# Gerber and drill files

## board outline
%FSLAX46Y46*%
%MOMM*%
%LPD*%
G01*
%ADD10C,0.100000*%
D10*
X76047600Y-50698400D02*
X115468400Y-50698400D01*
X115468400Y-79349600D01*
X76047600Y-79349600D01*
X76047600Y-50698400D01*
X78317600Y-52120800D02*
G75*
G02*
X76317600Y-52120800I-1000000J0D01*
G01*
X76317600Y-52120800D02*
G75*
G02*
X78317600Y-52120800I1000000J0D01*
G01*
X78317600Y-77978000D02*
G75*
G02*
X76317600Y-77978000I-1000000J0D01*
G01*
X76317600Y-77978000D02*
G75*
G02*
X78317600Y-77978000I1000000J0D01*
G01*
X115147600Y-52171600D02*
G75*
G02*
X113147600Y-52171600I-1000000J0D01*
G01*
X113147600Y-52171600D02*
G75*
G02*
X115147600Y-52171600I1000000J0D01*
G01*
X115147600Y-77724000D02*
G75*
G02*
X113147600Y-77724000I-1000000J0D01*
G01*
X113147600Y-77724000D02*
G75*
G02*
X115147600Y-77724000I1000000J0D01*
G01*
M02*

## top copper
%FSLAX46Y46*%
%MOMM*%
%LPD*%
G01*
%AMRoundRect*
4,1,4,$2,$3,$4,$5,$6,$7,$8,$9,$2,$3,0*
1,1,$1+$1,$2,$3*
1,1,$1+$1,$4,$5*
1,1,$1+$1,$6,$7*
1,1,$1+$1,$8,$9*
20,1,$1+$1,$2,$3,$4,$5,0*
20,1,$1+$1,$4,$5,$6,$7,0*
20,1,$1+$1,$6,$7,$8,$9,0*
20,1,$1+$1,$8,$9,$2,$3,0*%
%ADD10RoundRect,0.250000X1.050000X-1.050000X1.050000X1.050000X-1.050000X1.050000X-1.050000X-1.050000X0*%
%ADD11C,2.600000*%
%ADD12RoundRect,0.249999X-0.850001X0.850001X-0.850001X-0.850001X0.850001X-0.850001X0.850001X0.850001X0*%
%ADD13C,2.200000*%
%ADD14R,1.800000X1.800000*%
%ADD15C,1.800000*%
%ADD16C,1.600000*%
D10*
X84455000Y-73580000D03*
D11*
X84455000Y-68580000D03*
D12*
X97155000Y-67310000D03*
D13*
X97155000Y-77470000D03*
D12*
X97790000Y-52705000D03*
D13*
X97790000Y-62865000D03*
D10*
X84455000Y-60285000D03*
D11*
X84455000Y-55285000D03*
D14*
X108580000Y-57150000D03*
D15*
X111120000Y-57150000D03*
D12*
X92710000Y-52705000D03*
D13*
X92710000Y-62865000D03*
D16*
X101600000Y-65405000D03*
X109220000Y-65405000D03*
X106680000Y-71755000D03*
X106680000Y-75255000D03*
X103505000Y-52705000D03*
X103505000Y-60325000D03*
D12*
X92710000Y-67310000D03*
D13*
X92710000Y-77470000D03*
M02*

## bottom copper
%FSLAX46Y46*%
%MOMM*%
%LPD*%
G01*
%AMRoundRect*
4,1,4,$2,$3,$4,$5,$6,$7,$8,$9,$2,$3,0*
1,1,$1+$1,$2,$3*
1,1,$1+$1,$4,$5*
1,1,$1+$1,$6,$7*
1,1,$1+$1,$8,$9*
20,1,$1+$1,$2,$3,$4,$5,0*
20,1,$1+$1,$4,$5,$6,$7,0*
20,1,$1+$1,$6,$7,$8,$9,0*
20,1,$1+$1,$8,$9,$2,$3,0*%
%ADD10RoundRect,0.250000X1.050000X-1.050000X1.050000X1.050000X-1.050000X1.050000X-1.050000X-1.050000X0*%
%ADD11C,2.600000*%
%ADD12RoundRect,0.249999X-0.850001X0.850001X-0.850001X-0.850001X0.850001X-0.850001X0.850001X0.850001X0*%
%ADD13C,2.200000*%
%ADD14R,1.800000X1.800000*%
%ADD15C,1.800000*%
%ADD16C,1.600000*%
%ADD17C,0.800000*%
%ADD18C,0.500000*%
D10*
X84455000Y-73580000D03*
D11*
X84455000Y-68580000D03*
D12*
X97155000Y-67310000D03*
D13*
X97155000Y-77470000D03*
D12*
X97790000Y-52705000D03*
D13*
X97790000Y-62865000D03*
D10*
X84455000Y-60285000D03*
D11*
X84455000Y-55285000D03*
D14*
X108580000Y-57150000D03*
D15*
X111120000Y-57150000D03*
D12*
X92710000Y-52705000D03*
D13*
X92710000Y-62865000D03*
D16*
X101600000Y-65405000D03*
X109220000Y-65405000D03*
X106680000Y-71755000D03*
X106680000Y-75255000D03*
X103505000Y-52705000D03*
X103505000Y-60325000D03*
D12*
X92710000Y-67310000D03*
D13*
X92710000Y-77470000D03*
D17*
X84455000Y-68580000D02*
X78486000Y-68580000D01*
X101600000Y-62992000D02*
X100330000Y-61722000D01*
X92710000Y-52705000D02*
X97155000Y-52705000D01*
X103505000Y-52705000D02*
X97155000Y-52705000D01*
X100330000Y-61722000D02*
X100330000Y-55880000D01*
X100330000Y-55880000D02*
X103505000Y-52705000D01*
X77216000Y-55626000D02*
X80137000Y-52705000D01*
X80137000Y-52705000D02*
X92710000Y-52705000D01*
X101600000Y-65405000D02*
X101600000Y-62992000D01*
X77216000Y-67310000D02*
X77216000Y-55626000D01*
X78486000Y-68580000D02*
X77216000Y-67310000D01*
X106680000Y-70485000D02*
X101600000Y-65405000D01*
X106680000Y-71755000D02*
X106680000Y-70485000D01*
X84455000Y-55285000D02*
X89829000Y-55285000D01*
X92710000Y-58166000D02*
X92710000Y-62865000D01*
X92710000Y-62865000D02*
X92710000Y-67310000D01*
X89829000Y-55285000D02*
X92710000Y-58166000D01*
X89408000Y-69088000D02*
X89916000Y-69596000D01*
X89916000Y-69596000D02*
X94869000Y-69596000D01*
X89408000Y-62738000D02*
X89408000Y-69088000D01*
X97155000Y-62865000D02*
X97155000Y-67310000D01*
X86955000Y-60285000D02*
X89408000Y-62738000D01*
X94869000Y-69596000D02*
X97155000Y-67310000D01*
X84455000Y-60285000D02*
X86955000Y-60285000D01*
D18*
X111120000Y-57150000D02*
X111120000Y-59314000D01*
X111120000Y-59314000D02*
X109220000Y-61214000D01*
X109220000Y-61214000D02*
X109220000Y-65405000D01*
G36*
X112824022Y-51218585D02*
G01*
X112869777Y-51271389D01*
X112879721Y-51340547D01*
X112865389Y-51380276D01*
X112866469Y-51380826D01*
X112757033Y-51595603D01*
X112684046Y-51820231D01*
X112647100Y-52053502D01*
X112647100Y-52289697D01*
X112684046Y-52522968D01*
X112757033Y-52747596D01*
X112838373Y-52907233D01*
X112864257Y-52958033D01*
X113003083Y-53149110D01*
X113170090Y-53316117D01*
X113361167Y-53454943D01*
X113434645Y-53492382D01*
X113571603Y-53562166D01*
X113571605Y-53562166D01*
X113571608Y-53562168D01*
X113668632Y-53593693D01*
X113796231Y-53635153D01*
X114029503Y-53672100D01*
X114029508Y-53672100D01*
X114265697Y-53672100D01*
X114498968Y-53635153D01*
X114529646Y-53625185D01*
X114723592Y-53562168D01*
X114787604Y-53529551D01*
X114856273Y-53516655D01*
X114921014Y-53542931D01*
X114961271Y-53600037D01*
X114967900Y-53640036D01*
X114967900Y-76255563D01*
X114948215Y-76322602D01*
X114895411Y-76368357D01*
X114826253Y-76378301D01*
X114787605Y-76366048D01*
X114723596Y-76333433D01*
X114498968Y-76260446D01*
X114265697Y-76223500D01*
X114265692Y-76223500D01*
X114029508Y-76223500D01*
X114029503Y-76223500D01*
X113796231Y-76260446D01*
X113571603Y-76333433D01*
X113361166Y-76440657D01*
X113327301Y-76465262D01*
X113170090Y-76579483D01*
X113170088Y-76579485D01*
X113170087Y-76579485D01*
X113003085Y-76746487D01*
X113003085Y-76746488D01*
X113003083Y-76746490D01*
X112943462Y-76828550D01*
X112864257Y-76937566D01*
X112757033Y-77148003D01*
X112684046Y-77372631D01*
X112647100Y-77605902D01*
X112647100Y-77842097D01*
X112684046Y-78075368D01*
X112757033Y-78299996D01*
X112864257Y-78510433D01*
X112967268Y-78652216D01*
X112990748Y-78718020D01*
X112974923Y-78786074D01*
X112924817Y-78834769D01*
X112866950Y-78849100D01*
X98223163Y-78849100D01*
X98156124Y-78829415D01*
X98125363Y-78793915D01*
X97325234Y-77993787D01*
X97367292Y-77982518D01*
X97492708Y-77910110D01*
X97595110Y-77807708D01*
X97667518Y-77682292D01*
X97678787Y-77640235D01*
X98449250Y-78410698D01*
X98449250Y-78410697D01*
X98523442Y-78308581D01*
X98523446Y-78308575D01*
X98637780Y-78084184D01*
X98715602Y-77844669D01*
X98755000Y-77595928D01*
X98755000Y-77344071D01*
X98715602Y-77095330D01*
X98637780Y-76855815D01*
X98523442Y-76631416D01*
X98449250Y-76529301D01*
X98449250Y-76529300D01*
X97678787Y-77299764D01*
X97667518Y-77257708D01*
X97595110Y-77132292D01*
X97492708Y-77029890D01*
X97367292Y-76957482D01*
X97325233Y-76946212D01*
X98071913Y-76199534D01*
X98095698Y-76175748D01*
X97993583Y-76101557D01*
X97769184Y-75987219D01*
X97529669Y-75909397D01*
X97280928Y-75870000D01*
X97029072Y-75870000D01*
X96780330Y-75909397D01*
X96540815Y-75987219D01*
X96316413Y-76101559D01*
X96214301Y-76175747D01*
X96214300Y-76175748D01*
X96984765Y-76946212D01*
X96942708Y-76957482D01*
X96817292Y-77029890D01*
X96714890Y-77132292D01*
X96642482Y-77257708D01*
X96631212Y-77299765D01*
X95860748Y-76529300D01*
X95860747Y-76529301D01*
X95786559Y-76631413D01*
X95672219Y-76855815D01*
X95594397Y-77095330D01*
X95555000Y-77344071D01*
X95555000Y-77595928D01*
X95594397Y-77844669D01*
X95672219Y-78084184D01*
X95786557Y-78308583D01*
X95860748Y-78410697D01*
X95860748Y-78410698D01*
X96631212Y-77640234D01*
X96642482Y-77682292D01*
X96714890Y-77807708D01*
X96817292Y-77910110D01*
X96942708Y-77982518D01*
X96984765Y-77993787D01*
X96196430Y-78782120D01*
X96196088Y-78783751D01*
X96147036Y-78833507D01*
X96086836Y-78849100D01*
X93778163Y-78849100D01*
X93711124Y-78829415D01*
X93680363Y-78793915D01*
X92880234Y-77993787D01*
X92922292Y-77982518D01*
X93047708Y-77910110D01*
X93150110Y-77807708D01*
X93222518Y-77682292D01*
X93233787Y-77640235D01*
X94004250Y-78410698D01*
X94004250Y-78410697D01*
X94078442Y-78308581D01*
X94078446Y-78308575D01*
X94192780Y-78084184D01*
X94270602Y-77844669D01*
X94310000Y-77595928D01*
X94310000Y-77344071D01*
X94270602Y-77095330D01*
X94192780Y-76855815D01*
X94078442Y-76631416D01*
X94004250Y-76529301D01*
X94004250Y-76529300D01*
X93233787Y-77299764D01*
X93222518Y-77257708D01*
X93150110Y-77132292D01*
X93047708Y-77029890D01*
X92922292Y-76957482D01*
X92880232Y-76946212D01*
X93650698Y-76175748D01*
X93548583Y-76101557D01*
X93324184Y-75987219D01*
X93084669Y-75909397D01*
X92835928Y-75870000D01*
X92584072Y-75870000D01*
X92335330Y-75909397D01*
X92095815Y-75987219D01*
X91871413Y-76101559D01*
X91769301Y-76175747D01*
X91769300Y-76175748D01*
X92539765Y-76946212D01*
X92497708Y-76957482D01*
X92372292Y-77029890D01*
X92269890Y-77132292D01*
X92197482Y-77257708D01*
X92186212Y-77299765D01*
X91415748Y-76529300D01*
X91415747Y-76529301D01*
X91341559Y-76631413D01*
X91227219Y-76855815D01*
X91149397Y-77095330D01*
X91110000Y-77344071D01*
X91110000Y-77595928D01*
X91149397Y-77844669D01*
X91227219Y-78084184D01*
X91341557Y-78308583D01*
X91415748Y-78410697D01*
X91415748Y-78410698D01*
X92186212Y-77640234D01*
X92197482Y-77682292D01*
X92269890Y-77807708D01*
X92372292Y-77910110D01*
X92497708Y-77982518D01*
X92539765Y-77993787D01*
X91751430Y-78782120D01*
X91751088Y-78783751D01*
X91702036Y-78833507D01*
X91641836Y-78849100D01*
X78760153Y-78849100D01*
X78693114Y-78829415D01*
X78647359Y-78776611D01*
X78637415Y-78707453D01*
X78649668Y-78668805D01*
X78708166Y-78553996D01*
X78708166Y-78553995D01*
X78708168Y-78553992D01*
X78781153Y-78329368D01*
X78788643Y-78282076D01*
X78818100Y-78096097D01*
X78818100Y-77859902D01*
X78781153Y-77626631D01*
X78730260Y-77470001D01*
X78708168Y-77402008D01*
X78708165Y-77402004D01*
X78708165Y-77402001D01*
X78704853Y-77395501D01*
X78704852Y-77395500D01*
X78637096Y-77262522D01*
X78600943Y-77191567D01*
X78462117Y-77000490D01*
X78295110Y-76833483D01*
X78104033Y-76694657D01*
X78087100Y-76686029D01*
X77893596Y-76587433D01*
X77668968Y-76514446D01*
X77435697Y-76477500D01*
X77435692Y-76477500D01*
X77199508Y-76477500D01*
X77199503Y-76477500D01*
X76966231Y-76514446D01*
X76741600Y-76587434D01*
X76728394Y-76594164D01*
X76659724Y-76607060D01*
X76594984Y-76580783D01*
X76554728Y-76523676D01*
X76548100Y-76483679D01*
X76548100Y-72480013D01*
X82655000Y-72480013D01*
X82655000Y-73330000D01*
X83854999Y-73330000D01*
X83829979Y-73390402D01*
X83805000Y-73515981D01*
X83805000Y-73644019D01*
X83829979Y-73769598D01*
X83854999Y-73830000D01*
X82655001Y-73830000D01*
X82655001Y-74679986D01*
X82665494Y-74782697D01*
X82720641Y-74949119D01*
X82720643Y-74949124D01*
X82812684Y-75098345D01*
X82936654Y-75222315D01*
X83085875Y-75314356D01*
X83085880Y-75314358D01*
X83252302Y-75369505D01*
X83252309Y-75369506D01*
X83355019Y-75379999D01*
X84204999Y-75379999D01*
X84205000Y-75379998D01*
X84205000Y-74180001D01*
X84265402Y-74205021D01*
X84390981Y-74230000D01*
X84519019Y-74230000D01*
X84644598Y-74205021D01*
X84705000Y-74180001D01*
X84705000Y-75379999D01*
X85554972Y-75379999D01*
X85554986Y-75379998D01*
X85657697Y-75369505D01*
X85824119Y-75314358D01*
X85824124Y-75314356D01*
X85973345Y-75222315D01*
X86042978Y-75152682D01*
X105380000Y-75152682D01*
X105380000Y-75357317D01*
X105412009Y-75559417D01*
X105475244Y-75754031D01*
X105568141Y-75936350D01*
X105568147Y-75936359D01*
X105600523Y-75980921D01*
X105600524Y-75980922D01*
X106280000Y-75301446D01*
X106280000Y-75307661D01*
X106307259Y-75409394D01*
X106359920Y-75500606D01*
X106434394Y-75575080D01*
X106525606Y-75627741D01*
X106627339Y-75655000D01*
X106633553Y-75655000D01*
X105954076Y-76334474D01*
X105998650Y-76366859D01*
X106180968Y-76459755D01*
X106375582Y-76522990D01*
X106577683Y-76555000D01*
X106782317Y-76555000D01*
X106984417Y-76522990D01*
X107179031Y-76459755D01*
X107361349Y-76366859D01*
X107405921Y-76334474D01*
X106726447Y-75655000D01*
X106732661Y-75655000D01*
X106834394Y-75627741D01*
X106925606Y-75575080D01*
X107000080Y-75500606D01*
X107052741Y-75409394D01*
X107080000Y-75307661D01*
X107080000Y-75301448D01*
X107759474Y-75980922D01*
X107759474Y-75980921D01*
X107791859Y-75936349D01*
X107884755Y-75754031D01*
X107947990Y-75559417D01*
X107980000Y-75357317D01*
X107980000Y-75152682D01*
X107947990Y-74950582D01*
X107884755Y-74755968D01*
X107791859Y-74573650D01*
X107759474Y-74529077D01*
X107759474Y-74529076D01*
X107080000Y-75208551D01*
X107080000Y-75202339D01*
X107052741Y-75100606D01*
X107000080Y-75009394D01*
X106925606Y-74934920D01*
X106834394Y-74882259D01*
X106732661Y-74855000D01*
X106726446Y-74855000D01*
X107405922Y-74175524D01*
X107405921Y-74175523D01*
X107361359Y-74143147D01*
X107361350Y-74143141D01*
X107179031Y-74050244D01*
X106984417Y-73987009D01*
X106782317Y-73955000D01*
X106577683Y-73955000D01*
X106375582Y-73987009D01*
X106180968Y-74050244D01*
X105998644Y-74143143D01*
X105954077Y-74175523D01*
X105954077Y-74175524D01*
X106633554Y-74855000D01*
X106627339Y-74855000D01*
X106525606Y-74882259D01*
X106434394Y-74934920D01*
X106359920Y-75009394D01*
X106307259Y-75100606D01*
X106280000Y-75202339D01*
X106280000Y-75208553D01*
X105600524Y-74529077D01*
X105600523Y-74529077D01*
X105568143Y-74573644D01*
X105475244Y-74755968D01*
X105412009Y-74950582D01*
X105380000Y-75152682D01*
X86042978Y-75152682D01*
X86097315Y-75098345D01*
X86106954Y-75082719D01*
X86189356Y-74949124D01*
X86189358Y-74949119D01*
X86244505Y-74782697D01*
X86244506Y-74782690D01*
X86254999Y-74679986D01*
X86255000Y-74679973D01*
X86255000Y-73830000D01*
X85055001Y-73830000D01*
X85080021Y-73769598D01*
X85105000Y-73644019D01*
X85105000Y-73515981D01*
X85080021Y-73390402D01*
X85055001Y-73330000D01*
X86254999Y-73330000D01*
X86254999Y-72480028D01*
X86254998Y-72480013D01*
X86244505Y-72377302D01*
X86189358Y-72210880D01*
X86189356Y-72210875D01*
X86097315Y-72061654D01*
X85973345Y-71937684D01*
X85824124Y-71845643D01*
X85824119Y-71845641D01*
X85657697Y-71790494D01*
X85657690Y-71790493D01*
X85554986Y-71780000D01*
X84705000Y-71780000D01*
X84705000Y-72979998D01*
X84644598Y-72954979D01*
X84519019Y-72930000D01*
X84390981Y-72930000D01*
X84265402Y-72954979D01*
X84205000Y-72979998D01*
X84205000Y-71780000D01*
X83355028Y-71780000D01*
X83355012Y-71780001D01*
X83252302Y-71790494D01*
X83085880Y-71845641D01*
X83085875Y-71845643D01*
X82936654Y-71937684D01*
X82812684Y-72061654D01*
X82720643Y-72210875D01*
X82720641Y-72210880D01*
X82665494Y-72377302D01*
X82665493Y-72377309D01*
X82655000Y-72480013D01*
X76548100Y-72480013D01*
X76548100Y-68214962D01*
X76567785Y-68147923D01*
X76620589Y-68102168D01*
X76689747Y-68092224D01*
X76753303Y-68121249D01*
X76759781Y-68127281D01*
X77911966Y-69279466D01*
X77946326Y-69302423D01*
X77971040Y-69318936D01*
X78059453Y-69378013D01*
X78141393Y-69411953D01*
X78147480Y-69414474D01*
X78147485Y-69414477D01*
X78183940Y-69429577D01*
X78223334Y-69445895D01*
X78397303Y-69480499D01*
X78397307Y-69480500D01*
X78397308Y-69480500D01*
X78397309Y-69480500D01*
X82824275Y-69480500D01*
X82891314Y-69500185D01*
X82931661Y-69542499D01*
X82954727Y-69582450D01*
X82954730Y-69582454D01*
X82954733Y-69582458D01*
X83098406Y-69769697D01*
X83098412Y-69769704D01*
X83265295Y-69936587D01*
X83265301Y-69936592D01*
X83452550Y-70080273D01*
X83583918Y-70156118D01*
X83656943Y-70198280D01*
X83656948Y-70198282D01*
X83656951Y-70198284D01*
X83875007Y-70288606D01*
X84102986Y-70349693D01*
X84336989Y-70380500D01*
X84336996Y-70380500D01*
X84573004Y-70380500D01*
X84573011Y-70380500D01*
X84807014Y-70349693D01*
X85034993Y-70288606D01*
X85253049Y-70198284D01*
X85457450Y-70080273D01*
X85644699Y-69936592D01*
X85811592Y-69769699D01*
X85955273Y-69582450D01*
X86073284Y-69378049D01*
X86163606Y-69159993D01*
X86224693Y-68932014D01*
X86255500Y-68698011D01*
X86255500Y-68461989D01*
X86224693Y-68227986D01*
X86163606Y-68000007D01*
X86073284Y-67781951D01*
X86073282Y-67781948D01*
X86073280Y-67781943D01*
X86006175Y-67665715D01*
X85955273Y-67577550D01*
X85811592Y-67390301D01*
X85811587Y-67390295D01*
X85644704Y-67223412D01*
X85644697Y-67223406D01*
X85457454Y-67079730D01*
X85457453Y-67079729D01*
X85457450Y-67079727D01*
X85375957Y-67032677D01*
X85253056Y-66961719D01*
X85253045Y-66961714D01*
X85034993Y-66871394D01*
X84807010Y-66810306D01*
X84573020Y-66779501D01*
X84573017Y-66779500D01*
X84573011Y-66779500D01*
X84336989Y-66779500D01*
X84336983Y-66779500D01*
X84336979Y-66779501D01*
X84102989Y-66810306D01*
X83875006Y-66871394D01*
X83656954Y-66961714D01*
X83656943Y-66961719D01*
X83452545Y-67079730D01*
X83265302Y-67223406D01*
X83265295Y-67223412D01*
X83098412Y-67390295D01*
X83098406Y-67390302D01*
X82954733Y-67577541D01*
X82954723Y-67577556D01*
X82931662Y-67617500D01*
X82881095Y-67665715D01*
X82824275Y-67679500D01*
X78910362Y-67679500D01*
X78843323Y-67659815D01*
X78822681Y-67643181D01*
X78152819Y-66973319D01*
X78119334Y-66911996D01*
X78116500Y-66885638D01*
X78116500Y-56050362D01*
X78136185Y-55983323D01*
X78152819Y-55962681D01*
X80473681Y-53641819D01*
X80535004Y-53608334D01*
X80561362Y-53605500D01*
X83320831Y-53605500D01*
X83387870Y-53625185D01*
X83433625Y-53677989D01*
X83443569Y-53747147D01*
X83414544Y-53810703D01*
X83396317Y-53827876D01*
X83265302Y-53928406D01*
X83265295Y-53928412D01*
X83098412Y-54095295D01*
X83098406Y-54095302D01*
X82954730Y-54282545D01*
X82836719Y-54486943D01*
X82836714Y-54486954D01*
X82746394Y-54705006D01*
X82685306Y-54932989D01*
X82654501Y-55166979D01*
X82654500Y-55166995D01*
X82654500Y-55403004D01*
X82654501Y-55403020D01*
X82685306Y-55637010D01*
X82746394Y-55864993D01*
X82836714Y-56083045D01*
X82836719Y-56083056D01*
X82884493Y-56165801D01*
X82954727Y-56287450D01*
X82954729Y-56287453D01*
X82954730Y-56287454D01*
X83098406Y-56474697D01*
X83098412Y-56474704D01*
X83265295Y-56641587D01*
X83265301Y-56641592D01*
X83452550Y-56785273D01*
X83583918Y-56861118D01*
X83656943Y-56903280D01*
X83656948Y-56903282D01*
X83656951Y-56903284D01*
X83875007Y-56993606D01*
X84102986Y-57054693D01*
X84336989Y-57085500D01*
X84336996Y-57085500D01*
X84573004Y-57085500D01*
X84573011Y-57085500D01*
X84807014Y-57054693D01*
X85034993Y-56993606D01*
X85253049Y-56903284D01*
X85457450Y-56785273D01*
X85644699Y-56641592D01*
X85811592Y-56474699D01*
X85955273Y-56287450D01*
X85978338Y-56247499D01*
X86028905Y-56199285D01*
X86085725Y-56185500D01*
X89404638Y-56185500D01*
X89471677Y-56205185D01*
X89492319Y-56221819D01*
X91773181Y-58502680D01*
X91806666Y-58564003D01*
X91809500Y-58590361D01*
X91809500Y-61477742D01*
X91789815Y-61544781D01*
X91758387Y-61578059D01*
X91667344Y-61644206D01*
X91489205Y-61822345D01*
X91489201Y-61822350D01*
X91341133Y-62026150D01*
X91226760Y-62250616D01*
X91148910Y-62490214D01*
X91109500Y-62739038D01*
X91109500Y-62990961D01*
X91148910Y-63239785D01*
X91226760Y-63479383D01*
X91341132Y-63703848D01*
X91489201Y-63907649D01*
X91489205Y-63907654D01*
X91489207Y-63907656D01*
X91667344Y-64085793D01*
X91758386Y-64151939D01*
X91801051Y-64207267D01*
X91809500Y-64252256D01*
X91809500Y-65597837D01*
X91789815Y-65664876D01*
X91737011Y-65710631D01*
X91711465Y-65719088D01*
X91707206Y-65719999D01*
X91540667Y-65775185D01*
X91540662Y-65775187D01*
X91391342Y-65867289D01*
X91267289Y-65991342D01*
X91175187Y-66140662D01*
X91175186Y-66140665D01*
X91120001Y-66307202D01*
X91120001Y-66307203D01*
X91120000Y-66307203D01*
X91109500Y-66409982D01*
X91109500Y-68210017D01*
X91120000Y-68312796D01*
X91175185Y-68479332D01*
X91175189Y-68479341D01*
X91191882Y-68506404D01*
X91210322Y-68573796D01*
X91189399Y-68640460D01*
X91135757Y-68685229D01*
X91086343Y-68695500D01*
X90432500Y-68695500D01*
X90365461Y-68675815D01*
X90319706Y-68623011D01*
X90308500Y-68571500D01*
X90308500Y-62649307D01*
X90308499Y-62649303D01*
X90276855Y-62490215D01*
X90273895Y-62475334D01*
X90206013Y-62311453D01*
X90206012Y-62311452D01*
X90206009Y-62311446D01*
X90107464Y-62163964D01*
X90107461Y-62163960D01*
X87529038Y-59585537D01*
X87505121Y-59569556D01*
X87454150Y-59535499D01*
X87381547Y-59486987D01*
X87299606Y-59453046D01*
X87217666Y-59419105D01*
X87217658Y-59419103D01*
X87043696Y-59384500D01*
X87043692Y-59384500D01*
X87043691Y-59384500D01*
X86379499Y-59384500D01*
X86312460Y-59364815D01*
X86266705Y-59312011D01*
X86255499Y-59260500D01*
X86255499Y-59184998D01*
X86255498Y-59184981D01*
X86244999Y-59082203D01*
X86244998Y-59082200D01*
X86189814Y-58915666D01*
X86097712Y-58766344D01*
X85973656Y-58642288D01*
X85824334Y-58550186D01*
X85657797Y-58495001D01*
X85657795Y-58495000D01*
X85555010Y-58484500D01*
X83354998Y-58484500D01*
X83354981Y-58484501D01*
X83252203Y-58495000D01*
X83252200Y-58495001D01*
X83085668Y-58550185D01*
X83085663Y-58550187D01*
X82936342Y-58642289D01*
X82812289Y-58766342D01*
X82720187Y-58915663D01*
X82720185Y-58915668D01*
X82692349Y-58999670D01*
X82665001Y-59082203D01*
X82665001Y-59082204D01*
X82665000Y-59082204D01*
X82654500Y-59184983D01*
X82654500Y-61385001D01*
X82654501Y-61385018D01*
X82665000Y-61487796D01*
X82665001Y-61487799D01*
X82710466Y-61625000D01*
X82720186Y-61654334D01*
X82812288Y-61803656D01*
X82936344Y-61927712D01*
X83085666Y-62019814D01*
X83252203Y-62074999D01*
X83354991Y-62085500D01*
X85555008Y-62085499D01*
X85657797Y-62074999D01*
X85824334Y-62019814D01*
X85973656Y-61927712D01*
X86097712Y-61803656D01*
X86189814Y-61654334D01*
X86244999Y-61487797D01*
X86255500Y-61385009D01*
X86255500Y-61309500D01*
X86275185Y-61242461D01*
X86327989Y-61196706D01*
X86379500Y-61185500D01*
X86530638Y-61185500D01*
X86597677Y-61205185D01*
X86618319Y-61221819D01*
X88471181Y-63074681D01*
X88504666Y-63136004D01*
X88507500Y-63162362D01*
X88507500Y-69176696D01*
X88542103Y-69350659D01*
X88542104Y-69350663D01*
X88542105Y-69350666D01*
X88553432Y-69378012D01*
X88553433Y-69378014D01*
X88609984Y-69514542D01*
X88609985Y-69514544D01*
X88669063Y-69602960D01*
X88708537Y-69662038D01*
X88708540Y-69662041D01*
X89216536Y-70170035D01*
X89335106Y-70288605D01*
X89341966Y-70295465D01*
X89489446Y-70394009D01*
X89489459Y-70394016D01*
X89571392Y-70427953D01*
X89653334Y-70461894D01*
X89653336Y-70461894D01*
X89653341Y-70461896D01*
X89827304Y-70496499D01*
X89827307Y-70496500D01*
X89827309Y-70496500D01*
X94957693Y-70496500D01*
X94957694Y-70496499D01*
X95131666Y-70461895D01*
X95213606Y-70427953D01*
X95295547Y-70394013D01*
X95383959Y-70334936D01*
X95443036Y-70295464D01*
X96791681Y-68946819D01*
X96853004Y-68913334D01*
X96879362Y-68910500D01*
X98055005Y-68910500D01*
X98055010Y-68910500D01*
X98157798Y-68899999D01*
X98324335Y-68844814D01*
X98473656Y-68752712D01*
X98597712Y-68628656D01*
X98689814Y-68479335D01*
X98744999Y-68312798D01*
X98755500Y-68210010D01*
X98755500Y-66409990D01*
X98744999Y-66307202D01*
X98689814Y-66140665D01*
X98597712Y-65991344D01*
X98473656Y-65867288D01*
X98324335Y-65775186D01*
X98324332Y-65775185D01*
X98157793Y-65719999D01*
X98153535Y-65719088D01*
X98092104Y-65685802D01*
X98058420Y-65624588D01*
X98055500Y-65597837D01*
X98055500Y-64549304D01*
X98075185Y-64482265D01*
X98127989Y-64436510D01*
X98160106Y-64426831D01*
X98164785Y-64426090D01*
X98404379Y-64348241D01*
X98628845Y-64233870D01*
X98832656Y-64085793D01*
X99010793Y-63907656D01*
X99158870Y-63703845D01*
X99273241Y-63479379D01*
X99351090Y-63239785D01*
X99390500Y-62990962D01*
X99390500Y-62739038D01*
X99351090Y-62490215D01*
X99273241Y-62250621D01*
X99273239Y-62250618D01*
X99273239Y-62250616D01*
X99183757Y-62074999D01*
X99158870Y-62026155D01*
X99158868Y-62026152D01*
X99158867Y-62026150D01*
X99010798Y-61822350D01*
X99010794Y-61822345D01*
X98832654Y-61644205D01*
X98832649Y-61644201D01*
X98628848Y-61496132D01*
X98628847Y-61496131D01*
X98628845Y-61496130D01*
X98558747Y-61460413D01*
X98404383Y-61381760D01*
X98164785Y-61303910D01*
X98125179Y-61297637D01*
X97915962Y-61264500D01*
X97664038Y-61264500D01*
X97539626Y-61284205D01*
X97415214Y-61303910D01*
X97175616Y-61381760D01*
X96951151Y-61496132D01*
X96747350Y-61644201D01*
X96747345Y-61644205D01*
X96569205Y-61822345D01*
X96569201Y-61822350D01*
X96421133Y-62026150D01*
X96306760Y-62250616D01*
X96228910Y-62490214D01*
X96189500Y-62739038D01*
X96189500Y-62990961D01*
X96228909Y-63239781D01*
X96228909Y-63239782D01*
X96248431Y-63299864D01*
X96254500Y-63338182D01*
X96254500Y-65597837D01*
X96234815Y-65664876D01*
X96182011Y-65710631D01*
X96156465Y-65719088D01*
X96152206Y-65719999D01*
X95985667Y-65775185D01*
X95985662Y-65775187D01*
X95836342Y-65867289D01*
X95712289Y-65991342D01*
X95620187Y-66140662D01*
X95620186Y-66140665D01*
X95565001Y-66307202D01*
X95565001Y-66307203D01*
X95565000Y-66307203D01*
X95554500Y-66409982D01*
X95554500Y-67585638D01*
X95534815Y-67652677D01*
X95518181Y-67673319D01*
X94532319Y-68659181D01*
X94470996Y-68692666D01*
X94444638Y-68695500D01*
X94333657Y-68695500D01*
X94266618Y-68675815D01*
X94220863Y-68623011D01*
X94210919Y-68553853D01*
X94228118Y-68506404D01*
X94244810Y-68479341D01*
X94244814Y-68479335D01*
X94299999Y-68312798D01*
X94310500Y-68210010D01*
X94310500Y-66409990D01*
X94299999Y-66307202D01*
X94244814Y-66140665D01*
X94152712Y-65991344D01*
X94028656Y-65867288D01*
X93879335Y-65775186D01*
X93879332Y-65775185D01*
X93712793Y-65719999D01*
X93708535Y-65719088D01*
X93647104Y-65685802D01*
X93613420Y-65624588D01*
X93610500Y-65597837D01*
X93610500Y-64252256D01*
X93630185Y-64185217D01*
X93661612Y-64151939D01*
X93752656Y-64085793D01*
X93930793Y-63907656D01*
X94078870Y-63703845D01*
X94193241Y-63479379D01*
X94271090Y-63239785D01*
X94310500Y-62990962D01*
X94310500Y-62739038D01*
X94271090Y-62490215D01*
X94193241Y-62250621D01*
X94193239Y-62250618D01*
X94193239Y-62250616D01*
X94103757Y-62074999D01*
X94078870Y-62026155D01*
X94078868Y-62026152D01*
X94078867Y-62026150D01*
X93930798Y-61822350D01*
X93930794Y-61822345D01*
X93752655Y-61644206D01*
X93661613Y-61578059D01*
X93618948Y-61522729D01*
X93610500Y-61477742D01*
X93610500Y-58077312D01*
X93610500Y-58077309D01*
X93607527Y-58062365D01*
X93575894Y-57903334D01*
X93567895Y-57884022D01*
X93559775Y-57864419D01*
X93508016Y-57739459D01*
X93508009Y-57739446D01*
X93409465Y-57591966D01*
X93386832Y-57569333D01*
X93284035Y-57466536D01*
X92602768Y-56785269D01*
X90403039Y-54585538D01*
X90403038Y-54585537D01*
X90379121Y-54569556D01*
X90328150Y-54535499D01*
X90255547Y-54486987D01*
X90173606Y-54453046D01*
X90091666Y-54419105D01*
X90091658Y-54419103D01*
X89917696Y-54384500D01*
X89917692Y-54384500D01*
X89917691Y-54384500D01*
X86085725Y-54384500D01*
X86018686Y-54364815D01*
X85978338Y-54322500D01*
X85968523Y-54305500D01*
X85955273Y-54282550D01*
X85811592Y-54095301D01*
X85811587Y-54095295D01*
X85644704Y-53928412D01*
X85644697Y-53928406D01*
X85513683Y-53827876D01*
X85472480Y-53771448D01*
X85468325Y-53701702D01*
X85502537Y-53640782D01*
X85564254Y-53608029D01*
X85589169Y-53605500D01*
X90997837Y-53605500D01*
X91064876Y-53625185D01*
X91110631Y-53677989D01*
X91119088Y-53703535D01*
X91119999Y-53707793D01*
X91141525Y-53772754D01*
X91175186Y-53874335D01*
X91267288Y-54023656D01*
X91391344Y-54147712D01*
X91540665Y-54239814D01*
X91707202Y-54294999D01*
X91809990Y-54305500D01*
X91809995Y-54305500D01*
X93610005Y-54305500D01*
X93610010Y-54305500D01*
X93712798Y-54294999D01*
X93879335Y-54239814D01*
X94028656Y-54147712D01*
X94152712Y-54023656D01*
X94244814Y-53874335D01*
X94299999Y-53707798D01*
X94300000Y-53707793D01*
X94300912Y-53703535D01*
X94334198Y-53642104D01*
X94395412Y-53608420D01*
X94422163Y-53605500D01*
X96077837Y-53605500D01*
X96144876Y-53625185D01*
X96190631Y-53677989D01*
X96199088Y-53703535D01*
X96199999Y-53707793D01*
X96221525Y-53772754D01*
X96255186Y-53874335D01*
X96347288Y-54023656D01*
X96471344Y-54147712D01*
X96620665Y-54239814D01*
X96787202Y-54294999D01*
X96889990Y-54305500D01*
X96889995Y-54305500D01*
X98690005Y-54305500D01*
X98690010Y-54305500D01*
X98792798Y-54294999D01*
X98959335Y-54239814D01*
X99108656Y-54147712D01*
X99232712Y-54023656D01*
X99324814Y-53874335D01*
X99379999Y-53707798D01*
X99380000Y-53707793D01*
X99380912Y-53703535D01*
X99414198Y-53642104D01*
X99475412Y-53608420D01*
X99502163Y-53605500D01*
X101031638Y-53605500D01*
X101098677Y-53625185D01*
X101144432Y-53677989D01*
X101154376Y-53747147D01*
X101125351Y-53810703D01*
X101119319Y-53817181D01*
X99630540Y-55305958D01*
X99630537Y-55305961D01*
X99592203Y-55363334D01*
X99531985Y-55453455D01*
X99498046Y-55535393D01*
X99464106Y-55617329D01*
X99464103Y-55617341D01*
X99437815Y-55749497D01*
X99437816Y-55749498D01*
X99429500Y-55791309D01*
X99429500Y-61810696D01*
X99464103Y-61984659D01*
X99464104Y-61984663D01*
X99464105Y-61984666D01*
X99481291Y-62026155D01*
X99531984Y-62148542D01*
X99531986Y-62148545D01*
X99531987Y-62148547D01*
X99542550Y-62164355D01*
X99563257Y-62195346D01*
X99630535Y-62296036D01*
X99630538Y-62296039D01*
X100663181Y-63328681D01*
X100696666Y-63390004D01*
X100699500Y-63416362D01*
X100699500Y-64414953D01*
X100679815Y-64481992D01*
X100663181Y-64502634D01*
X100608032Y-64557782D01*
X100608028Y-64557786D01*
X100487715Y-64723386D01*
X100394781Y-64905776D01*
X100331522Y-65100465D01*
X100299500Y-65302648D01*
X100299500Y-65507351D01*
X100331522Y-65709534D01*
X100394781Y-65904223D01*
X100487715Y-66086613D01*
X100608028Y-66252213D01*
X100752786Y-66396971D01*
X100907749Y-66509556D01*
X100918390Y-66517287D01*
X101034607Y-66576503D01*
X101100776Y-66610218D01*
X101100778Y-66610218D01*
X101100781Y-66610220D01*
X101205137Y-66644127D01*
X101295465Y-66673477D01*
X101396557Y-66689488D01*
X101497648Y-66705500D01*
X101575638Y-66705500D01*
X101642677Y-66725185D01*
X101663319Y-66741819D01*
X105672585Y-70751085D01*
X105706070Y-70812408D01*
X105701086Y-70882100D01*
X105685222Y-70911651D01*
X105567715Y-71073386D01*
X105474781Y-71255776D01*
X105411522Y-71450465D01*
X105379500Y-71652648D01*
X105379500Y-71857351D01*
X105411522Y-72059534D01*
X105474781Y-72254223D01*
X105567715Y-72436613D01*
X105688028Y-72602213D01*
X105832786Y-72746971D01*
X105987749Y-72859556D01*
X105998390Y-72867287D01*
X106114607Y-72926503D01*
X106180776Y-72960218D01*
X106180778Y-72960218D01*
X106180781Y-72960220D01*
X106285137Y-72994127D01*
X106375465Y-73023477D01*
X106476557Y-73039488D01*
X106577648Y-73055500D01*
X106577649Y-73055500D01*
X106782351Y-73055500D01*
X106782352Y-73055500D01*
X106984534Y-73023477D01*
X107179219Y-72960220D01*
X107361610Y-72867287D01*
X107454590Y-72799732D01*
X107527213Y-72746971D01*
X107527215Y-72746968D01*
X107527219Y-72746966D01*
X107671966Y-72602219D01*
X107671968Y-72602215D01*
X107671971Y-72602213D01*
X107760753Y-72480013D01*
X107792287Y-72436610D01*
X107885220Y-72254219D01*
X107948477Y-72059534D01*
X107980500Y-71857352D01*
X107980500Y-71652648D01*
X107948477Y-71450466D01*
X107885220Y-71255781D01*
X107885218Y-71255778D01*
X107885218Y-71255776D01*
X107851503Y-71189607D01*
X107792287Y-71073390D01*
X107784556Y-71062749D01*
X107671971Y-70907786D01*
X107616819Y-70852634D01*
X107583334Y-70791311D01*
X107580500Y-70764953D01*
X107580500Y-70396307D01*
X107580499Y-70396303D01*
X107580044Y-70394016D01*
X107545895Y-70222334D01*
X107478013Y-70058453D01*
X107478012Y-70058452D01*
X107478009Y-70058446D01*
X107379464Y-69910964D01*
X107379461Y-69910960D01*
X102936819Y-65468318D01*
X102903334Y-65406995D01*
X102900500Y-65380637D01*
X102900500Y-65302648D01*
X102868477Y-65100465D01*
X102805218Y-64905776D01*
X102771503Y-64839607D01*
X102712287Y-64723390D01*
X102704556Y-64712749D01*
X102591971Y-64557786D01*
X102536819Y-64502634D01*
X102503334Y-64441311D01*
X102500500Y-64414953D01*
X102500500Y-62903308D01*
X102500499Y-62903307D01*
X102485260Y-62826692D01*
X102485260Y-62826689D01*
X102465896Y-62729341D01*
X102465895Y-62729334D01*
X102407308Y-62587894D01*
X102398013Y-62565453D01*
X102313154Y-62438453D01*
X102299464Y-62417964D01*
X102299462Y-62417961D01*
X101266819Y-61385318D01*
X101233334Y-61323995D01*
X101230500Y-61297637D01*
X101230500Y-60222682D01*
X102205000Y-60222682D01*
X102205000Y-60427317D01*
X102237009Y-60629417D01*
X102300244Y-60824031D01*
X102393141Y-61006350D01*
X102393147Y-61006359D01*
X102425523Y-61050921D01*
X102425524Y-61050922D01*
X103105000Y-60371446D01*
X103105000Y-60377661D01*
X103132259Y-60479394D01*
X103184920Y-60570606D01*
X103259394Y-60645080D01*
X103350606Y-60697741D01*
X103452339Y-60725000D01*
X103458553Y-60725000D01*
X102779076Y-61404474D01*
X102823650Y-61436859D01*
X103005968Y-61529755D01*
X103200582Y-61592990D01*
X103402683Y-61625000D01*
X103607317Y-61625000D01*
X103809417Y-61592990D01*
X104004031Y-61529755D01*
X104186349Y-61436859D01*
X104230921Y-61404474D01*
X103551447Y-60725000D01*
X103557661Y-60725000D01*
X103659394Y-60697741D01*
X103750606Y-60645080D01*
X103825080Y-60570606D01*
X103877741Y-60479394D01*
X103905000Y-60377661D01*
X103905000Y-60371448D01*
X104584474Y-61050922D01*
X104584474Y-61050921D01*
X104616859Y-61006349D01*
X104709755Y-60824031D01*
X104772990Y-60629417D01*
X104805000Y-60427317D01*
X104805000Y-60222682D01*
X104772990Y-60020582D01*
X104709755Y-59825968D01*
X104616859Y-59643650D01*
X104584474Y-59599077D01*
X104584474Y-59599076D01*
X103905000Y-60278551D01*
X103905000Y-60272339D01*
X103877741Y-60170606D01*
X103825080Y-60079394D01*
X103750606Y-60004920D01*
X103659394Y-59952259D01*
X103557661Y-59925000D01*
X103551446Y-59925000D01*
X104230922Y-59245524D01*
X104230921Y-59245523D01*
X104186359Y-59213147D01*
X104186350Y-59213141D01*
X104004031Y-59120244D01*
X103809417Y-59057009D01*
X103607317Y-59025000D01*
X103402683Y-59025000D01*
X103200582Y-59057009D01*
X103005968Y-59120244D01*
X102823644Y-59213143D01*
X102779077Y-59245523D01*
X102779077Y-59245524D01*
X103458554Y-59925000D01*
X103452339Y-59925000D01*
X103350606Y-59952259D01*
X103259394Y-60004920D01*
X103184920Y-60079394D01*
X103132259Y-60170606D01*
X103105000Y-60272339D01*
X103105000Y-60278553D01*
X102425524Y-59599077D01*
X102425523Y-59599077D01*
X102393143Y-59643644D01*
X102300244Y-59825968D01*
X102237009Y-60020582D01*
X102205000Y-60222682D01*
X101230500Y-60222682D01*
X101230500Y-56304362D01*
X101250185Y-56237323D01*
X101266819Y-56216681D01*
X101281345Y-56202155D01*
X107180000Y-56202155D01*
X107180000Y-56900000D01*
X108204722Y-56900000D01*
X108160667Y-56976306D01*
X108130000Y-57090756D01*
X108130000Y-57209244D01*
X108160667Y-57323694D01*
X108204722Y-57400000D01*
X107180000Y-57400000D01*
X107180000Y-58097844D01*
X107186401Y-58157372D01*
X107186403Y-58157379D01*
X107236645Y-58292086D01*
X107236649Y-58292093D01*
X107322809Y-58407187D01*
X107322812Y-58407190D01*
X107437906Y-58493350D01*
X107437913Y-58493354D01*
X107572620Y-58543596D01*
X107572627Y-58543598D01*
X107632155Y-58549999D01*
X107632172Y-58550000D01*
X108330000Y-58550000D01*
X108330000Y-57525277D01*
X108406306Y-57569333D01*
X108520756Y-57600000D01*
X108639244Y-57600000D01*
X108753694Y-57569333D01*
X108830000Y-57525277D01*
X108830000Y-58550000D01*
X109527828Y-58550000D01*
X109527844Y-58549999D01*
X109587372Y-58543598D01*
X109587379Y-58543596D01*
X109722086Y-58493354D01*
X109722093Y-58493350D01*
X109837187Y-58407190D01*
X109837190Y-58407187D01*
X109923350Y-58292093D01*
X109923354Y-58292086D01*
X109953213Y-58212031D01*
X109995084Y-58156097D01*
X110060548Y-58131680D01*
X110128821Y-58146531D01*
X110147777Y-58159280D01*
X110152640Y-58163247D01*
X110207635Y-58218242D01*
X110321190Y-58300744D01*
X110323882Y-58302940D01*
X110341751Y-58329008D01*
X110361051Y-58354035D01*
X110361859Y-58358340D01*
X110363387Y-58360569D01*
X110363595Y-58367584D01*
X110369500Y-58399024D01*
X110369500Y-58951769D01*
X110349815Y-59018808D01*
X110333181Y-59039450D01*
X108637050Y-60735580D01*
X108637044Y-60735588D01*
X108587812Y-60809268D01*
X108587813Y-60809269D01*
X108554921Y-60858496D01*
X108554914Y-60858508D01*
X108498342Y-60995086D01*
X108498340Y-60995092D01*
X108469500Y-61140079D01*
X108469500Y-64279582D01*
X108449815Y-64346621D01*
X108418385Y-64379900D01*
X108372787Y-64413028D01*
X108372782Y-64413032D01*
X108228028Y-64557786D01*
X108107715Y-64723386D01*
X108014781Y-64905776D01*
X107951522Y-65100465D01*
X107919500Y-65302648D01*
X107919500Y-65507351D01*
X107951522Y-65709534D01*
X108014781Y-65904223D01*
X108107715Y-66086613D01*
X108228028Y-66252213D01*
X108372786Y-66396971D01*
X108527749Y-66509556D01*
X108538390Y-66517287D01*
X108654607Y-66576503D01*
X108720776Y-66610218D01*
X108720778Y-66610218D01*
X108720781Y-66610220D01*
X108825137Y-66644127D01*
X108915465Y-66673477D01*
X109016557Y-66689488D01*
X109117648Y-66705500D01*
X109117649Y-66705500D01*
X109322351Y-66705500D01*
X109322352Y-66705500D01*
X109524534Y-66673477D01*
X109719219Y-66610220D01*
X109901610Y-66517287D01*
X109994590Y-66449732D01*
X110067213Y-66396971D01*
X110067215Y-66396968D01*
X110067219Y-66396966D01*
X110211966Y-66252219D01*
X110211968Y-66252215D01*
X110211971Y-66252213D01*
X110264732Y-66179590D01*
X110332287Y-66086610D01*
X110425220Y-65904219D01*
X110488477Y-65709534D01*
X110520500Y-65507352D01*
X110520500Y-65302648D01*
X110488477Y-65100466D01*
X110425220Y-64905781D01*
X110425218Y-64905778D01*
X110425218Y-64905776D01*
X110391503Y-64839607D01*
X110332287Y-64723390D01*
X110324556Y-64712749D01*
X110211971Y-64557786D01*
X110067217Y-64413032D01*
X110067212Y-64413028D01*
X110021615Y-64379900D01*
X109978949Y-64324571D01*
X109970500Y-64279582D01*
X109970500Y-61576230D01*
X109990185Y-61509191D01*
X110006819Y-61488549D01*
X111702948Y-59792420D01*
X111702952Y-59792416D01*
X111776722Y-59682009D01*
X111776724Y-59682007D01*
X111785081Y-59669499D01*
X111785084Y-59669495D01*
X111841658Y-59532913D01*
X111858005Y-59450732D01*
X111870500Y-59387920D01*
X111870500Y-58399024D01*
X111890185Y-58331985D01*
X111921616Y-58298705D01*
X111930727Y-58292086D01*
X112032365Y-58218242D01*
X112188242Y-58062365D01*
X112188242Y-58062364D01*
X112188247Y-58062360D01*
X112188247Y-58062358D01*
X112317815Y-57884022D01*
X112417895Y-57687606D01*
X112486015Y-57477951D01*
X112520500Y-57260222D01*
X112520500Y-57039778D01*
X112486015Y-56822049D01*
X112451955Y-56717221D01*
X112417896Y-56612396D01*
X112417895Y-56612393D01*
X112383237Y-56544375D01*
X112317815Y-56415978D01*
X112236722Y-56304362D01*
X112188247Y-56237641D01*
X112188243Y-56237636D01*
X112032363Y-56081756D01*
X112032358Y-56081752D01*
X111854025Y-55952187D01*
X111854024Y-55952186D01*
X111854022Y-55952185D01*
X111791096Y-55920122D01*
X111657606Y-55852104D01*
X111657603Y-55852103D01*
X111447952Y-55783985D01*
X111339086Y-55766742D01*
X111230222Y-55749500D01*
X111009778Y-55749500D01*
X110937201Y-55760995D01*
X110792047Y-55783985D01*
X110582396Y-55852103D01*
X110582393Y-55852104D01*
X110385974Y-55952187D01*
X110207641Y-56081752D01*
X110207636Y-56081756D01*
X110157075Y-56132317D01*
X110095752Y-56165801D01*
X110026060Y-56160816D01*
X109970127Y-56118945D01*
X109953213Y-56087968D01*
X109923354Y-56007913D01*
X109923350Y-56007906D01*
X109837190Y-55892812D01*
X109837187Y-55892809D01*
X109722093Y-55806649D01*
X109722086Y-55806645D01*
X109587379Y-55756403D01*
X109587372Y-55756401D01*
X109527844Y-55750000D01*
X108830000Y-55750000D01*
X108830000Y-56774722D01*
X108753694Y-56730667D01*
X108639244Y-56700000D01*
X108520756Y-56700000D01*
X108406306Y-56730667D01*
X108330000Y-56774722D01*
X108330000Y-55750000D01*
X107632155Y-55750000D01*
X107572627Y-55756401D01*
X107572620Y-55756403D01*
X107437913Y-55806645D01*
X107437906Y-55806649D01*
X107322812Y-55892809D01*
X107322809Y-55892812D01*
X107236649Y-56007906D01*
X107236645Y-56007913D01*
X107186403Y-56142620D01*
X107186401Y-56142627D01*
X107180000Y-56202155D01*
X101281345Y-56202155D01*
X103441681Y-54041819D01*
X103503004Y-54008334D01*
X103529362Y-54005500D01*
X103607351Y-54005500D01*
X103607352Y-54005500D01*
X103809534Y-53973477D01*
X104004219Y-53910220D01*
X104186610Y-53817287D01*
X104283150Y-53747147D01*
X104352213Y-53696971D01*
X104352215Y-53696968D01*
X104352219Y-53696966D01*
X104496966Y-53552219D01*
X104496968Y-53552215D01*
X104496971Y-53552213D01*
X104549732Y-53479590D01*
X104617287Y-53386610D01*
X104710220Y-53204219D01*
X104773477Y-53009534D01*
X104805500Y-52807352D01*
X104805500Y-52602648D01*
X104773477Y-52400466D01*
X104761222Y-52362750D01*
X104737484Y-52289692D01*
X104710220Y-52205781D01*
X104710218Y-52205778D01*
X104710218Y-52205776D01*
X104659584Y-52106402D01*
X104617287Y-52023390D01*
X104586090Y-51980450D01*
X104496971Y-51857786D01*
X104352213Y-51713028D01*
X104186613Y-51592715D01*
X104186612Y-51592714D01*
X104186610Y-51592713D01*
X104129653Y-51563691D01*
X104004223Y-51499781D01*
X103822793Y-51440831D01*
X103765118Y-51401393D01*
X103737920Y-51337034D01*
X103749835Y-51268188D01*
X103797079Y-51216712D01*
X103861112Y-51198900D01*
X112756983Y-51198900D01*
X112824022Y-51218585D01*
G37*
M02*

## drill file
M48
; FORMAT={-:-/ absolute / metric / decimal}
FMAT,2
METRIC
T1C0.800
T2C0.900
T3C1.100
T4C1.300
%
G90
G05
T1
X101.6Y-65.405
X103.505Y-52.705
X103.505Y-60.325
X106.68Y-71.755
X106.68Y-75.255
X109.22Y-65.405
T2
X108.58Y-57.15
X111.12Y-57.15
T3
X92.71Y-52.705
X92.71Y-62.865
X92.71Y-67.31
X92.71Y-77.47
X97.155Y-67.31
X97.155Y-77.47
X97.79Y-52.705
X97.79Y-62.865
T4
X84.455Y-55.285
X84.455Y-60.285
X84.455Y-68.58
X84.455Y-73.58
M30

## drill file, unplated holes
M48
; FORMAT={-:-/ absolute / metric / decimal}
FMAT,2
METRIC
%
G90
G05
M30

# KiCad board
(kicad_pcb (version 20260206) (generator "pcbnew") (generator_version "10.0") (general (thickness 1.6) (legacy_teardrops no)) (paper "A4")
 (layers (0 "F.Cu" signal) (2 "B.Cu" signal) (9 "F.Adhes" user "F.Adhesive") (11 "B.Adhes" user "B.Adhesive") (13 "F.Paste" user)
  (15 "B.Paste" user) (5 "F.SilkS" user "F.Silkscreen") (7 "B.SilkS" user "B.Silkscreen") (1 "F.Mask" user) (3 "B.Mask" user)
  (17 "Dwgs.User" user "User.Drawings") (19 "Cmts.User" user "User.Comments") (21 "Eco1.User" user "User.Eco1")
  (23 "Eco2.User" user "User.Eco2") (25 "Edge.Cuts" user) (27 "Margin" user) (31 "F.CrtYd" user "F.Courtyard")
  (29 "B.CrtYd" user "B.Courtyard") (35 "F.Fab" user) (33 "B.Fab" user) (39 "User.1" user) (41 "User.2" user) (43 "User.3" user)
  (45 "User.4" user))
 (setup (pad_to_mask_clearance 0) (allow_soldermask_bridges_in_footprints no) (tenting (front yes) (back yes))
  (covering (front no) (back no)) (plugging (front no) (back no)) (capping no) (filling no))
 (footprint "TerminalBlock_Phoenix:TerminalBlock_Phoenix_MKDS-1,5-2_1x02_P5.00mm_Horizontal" (layer "F.Cu") (at 84.455 73.58 90)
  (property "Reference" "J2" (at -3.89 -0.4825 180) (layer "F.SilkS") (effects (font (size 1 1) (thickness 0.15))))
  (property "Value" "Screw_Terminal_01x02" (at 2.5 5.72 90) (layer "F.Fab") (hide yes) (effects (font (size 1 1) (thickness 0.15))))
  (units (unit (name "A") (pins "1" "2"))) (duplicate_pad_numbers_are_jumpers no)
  (pad "1" thru_hole roundrect (at 0 0 90) (size 2.6 2.6) (drill 1.3) (layers "*.Cu" "*.Mask") (remove_unused_layers no)
   (roundrect_rratio 0.096154) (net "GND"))
  (pad "2" thru_hole circle (at 5 0 90) (size 2.6 2.6) (drill 1.3) (layers "*.Cu" "*.Mask") (remove_unused_layers no) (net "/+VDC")))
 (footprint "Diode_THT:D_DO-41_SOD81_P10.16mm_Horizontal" (layer "F.Cu") (at 97.155 67.31 -90)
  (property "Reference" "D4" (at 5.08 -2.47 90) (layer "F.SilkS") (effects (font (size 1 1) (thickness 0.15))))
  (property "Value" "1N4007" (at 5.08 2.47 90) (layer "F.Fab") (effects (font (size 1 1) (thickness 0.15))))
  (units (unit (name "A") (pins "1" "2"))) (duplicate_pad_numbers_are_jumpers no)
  (pad "1" thru_hole roundrect (at 0 0 270) (size 2.2 2.2) (drill 1.1) (layers "*.Cu" "*.Mask") (remove_unused_layers no)
   (roundrect_rratio 0.113636) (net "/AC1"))
  (pad "2" thru_hole circle (at 10.16 0 270) (size 2.2 2.2) (drill 1.1) (layers "*.Cu" "*.Mask") (remove_unused_layers no) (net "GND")))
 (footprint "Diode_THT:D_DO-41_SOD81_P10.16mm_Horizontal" (layer "F.Cu") (at 97.79 52.705 -90)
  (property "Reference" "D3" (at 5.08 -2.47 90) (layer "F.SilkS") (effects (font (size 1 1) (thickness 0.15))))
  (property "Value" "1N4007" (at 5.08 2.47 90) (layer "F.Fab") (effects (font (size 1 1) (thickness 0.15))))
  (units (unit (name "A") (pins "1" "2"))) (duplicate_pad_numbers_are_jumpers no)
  (pad "1" thru_hole roundrect (at 0 0 270) (size 2.2 2.2) (drill 1.1) (layers "*.Cu" "*.Mask") (remove_unused_layers no)
   (roundrect_rratio 0.113636) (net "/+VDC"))
  (pad "2" thru_hole circle (at 10.16 0 270) (size 2.2 2.2) (drill 1.1) (layers "*.Cu" "*.Mask") (remove_unused_layers no) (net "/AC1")))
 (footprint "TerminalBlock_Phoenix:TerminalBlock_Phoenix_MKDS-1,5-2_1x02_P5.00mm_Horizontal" (layer "F.Cu") (at 84.455 60.285 90)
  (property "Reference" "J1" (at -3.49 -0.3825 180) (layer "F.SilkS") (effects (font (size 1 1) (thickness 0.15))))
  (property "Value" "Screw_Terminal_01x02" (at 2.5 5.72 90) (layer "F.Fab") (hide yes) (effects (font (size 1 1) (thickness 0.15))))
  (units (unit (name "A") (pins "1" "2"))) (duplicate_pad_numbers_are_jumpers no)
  (pad "1" thru_hole roundrect (at 0 0 90) (size 2.6 2.6) (drill 1.3) (layers "*.Cu" "*.Mask") (remove_unused_layers no)
   (roundrect_rratio 0.096154) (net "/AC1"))
  (pad "2" thru_hole circle (at 5 0 90) (size 2.6 2.6) (drill 1.3) (layers "*.Cu" "*.Mask") (remove_unused_layers no) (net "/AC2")))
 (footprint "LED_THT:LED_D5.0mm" (layer "F.Cu") (at 108.58 57.15)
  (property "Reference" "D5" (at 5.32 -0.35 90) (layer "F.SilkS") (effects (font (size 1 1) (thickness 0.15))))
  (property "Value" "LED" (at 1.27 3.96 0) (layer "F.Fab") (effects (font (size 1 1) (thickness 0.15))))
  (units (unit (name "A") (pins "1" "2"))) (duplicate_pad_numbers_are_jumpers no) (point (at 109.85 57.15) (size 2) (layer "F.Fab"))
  (pad "1" thru_hole rect (at 0 0) (size 1.8 1.8) (drill 0.9) (layers "*.Cu" "*.Mask") (remove_unused_layers no) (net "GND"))
  (pad "2" thru_hole circle (at 2.54 0) (size 1.8 1.8) (drill 0.9) (layers "*.Cu" "*.Mask") (remove_unused_layers no) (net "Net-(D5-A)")))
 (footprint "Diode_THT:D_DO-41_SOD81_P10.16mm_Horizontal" (layer "F.Cu") (at 92.71 52.705 -90)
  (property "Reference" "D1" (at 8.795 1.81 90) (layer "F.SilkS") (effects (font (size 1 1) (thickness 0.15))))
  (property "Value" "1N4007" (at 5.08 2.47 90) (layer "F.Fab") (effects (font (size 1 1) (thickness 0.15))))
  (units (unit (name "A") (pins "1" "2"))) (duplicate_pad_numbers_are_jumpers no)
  (pad "1" thru_hole roundrect (at 0 0 270) (size 2.2 2.2) (drill 1.1) (layers "*.Cu" "*.Mask") (remove_unused_layers no)
   (roundrect_rratio 0.113636) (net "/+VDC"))
  (pad "2" thru_hole circle (at 10.16 0 270) (size 2.2 2.2) (drill 1.1) (layers "*.Cu" "*.Mask") (remove_unused_layers no) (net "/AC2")))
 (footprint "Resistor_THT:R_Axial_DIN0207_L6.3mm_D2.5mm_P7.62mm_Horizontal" (layer "F.Cu") (at 101.6 65.405)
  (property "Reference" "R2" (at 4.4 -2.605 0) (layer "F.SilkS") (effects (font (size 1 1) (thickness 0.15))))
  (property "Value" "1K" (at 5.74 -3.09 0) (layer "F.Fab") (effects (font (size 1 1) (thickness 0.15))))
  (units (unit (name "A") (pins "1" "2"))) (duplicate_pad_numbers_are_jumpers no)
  (pad "1" thru_hole circle (at 0 0) (size 1.6 1.6) (drill 0.8) (layers "*.Cu" "*.Mask") (remove_unused_layers no) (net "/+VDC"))
  (pad "2" thru_hole circle (at 7.62 0) (size 1.6 1.6) (drill 0.8) (layers "*.Cu" "*.Mask") (remove_unused_layers no) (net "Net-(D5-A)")))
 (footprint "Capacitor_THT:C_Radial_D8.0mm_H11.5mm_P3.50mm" (layer "F.Cu") (at 106.68 71.755 -90)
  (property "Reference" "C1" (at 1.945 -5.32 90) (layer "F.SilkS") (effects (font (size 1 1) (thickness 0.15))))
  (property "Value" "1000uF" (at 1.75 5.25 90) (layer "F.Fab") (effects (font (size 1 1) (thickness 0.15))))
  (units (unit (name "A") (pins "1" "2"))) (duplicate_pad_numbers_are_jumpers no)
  (pad "1" thru_hole circle (at 0 0 270) (size 1.6 1.6) (drill 0.8) (layers "*.Cu" "*.Mask") (remove_unused_layers no) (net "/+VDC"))
  (pad "2" thru_hole circle (at 3.5 0 270) (size 1.6 1.6) (drill 0.8) (layers "*.Cu" "*.Mask") (remove_unused_layers no) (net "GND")))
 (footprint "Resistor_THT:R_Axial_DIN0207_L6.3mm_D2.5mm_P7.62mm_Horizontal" (layer "F.Cu") (at 103.505 52.705 -90)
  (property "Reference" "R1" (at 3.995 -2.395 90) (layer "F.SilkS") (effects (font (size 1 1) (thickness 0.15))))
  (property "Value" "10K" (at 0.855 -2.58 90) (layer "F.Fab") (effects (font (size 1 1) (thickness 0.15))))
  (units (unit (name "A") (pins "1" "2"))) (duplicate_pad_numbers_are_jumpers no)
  (pad "1" thru_hole circle (at 0 0 270) (size 1.6 1.6) (drill 0.8) (layers "*.Cu" "*.Mask") (remove_unused_layers no) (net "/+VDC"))
  (pad "2" thru_hole circle (at 7.62 0 270) (size 1.6 1.6) (drill 0.8) (layers "*.Cu" "*.Mask") (remove_unused_layers no) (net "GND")))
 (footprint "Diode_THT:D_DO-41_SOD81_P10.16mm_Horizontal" (layer "F.Cu") (at 92.71 67.31 -90)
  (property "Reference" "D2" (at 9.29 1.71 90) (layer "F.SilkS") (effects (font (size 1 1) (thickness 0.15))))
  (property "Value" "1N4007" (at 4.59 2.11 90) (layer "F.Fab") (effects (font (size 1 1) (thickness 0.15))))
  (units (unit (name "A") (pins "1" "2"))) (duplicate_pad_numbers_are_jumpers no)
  (pad "1" thru_hole roundrect (at 0 0 270) (size 2.2 2.2) (drill 1.1) (layers "*.Cu" "*.Mask") (remove_unused_layers no)
   (roundrect_rratio 0.113636) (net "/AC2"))
  (pad "2" thru_hole circle (at 10.16 0 270) (size 2.2 2.2) (drill 1.1) (layers "*.Cu" "*.Mask") (remove_unused_layers no) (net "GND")))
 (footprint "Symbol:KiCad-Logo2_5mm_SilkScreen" (layer "B.Cu") (at 94.234 72.898 180)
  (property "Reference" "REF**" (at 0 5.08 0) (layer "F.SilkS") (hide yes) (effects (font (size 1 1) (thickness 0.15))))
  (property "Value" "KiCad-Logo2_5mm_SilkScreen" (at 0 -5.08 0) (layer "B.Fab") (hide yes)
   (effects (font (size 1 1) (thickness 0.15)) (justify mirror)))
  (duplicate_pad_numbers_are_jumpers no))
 (gr_rect (start 76.0476 50.6984) (end 115.4684 79.3496) (stroke (width 0.1) (type solid)) (fill no) (layer "Edge.Cuts"))
 (gr_circle (center 77.3176 52.1208) (end 78.3176 52.1208) (stroke (width 0.1) (type solid)) (fill no) (layer "Edge.Cuts"))
 (gr_circle (center 77.3176 77.978) (end 78.3176 77.978) (stroke (width 0.1) (type solid)) (fill no) (layer "Edge.Cuts"))
 (gr_circle (center 114.1476 52.1716) (end 115.1476 52.1716) (stroke (width 0.1) (type solid)) (fill no) (layer "Edge.Cuts"))
 (gr_circle (center 114.1476 77.724) (end 115.1476 77.724) (stroke (width 0.1) (type solid)) (fill no) (layer "Edge.Cuts"))
 (segment (start 84.455 68.58) (end 78.486 68.58) (width 0.8) (layer "B.Cu") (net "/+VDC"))
 (segment (start 101.6 62.992) (end 100.33 61.722) (width 0.8) (layer "B.Cu") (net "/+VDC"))
 (segment (start 92.71 52.705) (end 97.155 52.705) (width 0.8) (layer "B.Cu") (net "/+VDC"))
 (segment (start 103.505 52.705) (end 97.155 52.705) (width 0.8) (layer "B.Cu") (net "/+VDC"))
 (segment (start 100.33 61.722) (end 100.33 55.88) (width 0.8) (layer "B.Cu") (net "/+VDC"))
 (segment (start 100.33 55.88) (end 103.505 52.705) (width 0.8) (layer "B.Cu") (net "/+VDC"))
 (segment (start 77.216 55.626) (end 80.137 52.705) (width 0.8) (layer "B.Cu") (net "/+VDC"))
 (segment (start 80.137 52.705) (end 92.71 52.705) (width 0.8) (layer "B.Cu") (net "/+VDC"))
 (segment (start 101.6 65.405) (end 101.6 62.992) (width 0.8) (layer "B.Cu") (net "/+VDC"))
 (segment (start 77.216 67.31) (end 77.216 55.626) (width 0.8) (layer "B.Cu") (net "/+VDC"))
 (segment (start 78.486 68.58) (end 77.216 67.31) (width 0.8) (layer "B.Cu") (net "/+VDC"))
 (segment (start 106.68 70.485) (end 101.6 65.405) (width 0.8) (layer "B.Cu") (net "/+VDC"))
 (segment (start 106.68 71.755) (end 106.68 70.485) (width 0.8) (layer "B.Cu") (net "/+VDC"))
 (segment (start 89.408 69.088) (end 89.916 69.596) (width 0.8) (layer "B.Cu") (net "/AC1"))
 (segment (start 89.916 69.596) (end 94.869 69.596) (width 0.8) (layer "B.Cu") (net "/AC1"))
 (segment (start 89.408 62.738) (end 89.408 69.088) (width 0.8) (layer "B.Cu") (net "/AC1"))
 (segment (start 97.155 62.865) (end 97.155 67.31) (width 0.8) (layer "B.Cu") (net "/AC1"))
 (segment (start 86.955 60.285) (end 89.408 62.738) (width 0.8) (layer "B.Cu") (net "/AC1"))
 (segment (start 94.869 69.596) (end 97.155 67.31) (width 0.8) (layer "B.Cu") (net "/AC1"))
 (segment (start 84.455 60.285) (end 86.955 60.285) (width 0.8) (layer "B.Cu") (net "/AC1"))
 (segment (start 84.455 55.285) (end 89.829 55.285) (width 0.8) (layer "B.Cu") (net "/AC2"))
 (segment (start 92.71 58.166) (end 92.71 62.865) (width 0.8) (layer "B.Cu") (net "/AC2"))
 (segment (start 92.71 62.865) (end 92.71 67.31) (width 0.8) (layer "B.Cu") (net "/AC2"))
 (segment (start 89.829 55.285) (end 92.71 58.166) (width 0.8) (layer "B.Cu") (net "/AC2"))
 (segment (start 111.12 57.15) (end 111.12 59.314) (width 0.5) (layer "B.Cu") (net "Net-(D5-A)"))
 (segment (start 111.12 59.314) (end 109.22 61.214) (width 0.5) (layer "B.Cu") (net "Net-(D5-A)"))
 (segment (start 109.22 61.214) (end 109.22 65.405) (width 0.5) (layer "B.Cu") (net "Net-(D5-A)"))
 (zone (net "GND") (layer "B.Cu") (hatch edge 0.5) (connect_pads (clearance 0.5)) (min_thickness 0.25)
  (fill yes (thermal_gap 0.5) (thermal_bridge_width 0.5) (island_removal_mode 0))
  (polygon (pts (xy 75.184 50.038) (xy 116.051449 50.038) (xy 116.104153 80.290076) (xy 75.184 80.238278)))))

